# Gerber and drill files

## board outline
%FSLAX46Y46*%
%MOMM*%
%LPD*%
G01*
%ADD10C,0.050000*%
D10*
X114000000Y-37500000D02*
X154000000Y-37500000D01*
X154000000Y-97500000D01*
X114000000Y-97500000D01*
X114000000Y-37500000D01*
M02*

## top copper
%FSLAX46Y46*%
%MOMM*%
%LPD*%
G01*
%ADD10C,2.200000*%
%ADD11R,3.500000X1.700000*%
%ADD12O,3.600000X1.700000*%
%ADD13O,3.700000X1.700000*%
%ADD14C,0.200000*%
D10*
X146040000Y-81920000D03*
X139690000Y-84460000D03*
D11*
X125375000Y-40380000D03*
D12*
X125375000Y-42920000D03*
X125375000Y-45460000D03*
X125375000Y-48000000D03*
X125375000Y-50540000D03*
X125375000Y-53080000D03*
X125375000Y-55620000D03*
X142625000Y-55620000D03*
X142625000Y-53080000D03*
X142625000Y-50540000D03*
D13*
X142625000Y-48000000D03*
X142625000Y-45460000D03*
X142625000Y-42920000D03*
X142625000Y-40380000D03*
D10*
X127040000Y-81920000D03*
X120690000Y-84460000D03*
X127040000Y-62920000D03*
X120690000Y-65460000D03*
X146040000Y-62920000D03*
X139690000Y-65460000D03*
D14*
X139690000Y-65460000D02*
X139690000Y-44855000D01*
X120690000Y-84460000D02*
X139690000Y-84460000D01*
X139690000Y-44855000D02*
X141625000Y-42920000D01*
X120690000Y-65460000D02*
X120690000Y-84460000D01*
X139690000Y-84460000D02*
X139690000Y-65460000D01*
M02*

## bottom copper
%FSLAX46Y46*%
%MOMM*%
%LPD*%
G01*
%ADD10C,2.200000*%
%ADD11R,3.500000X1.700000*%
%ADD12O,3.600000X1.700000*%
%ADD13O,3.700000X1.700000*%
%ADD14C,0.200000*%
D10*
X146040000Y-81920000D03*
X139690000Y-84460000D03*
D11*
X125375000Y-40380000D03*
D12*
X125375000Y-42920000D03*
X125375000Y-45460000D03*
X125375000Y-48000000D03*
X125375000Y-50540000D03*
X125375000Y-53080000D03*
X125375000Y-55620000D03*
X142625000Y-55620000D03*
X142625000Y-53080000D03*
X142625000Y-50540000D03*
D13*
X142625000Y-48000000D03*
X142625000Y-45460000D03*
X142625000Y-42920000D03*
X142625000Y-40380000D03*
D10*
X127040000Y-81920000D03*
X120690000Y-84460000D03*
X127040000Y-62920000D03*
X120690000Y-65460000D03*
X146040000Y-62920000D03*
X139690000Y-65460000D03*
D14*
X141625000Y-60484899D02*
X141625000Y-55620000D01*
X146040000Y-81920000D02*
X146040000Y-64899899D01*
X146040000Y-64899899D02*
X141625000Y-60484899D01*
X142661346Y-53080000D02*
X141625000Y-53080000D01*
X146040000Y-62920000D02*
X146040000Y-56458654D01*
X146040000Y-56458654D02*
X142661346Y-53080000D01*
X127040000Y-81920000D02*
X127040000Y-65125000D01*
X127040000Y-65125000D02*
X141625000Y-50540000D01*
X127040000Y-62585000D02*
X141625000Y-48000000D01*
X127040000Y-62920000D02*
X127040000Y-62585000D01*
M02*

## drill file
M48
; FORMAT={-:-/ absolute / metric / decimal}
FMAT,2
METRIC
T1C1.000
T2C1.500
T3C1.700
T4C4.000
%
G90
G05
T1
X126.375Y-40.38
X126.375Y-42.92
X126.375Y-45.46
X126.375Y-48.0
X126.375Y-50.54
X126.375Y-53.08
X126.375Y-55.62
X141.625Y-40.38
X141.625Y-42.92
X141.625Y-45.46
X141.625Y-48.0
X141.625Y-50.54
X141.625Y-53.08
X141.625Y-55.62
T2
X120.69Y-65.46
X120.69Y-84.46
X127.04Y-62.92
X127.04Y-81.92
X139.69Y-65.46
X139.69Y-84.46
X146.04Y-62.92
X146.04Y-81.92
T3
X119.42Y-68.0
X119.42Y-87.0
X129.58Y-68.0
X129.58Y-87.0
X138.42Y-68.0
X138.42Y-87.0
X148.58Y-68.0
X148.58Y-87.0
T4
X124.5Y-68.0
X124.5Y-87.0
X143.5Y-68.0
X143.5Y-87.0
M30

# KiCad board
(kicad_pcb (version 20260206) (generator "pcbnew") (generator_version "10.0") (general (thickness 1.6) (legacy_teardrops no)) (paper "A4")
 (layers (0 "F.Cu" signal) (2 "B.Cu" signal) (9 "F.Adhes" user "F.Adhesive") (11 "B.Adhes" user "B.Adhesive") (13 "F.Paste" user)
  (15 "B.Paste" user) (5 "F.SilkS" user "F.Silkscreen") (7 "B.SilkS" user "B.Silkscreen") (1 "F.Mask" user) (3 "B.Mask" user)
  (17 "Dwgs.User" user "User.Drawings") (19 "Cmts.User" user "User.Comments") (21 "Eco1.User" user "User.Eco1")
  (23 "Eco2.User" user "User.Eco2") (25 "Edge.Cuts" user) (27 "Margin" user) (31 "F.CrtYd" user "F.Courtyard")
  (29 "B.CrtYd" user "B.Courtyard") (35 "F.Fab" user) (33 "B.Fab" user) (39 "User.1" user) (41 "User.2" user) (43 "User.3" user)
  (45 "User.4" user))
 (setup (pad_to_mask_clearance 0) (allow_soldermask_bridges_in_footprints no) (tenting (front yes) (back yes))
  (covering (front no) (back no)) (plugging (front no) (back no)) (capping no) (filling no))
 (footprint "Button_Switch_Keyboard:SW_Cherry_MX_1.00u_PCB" (layer "F.Cu") (at 146.04 81.92)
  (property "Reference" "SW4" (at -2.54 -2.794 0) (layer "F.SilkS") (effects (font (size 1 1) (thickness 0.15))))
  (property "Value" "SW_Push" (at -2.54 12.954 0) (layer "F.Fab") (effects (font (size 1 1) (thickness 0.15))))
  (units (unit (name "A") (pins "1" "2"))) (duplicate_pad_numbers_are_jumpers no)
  (pad "" np_thru_hole circle (at -7.62 5.08) (size 1.7 1.7) (drill 1.7) (layers "*.Cu" "*.Mask"))
  (pad "" np_thru_hole circle (at -2.54 5.08) (size 4 4) (drill 4) (layers "*.Cu" "*.Mask"))
  (pad "" np_thru_hole circle (at 2.54 5.08) (size 1.7 1.7) (drill 1.7) (layers "*.Cu" "*.Mask"))
  (pad "1" thru_hole circle (at 0 0) (size 2.2 2.2) (drill 1.5) (layers "*.Cu" "*.Mask") (remove_unused_layers no)
   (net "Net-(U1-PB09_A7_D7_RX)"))
  (pad "2" thru_hole circle (at -6.35 2.54) (size 2.2 2.2) (drill 1.5) (layers "*.Cu" "*.Mask") (remove_unused_layers no) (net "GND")))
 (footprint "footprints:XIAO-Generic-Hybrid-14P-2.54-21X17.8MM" (layer "F.Cu") (at 134 48)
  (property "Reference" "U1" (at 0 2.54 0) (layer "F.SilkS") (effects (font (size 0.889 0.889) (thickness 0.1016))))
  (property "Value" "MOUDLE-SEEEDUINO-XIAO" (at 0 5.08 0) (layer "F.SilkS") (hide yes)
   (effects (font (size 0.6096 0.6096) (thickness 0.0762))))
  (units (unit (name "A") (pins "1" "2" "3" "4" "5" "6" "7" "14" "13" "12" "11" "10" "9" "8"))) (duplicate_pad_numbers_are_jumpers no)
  (pad "1" thru_hole rect (at -7.625 -7.62) (size 3.5 1.7) (drill 1 (offset -1 0)) (layers "*.Cu" "*.Mask") (remove_unused_layers no)
   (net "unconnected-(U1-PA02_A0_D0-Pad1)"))
  (pad "2" thru_hole oval (at -7.625 -5.08) (size 3.6 1.7) (drill 1 (offset -1 0)) (layers "*.Cu" "*.Mask") (remove_unused_layers no)
   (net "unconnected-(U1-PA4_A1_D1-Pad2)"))
  (pad "3" thru_hole oval (at -7.625 -2.54) (size 3.6 1.7) (drill 1 (offset -1 0)) (layers "*.Cu" "*.Mask") (remove_unused_layers no)
   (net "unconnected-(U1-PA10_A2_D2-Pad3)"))
  (pad "4" thru_hole oval (at -7.625 0) (size 3.6 1.7) (drill 1 (offset -1 0)) (layers "*.Cu" "*.Mask") (remove_unused_layers no)
   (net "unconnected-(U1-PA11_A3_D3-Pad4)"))
  (pad "5" thru_hole oval (at -7.625 2.54) (size 3.6 1.7) (drill 1 (offset -1 0)) (layers "*.Cu" "*.Mask") (remove_unused_layers no)
   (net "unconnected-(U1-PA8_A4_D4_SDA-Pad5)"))
  (pad "6" thru_hole oval (at -7.625 5.08 180) (size 3.6 1.7) (drill 1 (offset 1 0)) (layers "*.Cu" "*.Mask") (remove_unused_layers no)
   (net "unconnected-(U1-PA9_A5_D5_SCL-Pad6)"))
  (pad "7" thru_hole oval (at -7.625 7.62) (size 3.6 1.7) (drill 1 (offset -1 0)) (layers "*.Cu" "*.Mask") (remove_unused_layers no)
   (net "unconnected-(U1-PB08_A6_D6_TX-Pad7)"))
  (pad "8" thru_hole oval (at 7.625 7.62) (size 3.6 1.7) (drill 1 (offset 1 0)) (layers "*.Cu" "*.Mask") (remove_unused_layers no)
   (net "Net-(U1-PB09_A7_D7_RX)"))
  (pad "9" thru_hole oval (at 7.625 5.08) (size 3.6 1.7) (drill 1 (offset 1 0)) (layers "*.Cu" "*.Mask") (remove_unused_layers no)
   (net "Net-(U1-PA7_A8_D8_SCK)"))
  (pad "10" thru_hole oval (at 7.625 2.54) (size 3.6 1.7) (drill 1 (offset 1 0)) (layers "*.Cu" "*.Mask") (remove_unused_layers no)
   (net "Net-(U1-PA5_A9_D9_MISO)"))
  (pad "11" thru_hole oval (at 7.625 0) (size 3.7 1.7) (drill 1 (offset 1 0)) (layers "*.Cu" "*.Mask") (remove_unused_layers no)
   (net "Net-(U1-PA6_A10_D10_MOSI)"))
  (pad "12" thru_hole oval (at 7.625 -2.54) (size 3.7 1.7) (drill 1 (offset 1 0)) (layers "*.Cu" "*.Mask") (remove_unused_layers no)
   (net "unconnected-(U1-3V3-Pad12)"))
  (pad "13" thru_hole oval (at 7.625 -5.08) (size 3.7 1.7) (drill 1 (offset 1 0)) (layers "*.Cu" "*.Mask") (remove_unused_layers no)
   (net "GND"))
  (pad "14" thru_hole oval (at 7.625 -7.62) (size 3.7 1.7) (drill 1 (offset 1 0)) (layers "*.Cu" "*.Mask") (remove_unused_layers no)
   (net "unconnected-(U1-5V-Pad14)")))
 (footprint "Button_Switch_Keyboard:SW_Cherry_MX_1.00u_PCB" (layer "F.Cu") (at 127.04 81.92)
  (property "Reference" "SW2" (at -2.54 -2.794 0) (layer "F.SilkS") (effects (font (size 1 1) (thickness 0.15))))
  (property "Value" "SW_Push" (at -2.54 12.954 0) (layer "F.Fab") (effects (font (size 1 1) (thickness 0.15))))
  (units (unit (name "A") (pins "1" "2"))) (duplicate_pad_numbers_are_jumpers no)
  (pad "" np_thru_hole circle (at -7.62 5.08) (size 1.7 1.7) (drill 1.7) (layers "*.Cu" "*.Mask"))
  (pad "" np_thru_hole circle (at -2.54 5.08) (size 4 4) (drill 4) (layers "*.Cu" "*.Mask"))
  (pad "" np_thru_hole circle (at 2.54 5.08) (size 1.7 1.7) (drill 1.7) (layers "*.Cu" "*.Mask"))
  (pad "1" thru_hole circle (at 0 0) (size 2.2 2.2) (drill 1.5) (layers "*.Cu" "*.Mask") (remove_unused_layers no)
   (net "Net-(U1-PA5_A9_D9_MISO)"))
  (pad "2" thru_hole circle (at -6.35 2.54) (size 2.2 2.2) (drill 1.5) (layers "*.Cu" "*.Mask") (remove_unused_layers no) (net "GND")))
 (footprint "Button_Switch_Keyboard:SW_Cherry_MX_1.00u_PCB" (layer "F.Cu") (at 127.04 62.92)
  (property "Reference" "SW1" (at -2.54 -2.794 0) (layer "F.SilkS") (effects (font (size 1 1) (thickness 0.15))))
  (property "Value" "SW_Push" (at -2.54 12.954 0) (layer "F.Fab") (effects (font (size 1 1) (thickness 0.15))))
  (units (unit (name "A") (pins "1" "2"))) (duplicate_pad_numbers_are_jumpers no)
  (pad "" np_thru_hole circle (at -7.62 5.08) (size 1.7 1.7) (drill 1.7) (layers "*.Cu" "*.Mask"))
  (pad "" np_thru_hole circle (at -2.54 5.08) (size 4 4) (drill 4) (layers "*.Cu" "*.Mask"))
  (pad "" np_thru_hole circle (at 2.54 5.08) (size 1.7 1.7) (drill 1.7) (layers "*.Cu" "*.Mask"))
  (pad "1" thru_hole circle (at 0 0) (size 2.2 2.2) (drill 1.5) (layers "*.Cu" "*.Mask") (remove_unused_layers no)
   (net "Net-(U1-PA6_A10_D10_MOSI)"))
  (pad "2" thru_hole circle (at -6.35 2.54) (size 2.2 2.2) (drill 1.5) (layers "*.Cu" "*.Mask") (remove_unused_layers no) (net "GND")))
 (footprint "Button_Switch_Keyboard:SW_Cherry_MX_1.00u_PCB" (layer "F.Cu") (at 146.04 62.92)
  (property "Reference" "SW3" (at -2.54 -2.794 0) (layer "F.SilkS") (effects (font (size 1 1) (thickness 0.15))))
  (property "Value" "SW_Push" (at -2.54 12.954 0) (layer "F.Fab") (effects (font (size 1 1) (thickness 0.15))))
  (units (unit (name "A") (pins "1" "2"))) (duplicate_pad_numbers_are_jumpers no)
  (pad "" np_thru_hole circle (at -7.62 5.08) (size 1.7 1.7) (drill 1.7) (layers "*.Cu" "*.Mask"))
  (pad "" np_thru_hole circle (at -2.54 5.08) (size 4 4) (drill 4) (layers "*.Cu" "*.Mask"))
  (pad "" np_thru_hole circle (at 2.54 5.08) (size 1.7 1.7) (drill 1.7) (layers "*.Cu" "*.Mask"))
  (pad "1" thru_hole circle (at 0 0) (size 2.2 2.2) (drill 1.5) (layers "*.Cu" "*.Mask") (remove_unused_layers no)
   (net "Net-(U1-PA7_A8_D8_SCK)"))
  (pad "2" thru_hole circle (at -6.35 2.54) (size 2.2 2.2) (drill 1.5) (layers "*.Cu" "*.Mask") (remove_unused_layers no) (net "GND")))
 (gr_rect (start 114 37.5) (end 154 97.5) (stroke (width 0.05) (type default)) (fill no) (layer "Edge.Cuts"))
 (segment (start 141.625 60.484899) (end 141.625 55.62) (width 0.2) (layer "B.Cu") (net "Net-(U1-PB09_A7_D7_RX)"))
 (segment (start 146.04 81.92) (end 146.04 64.899899) (width 0.2) (layer "B.Cu") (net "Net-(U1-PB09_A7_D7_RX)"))
 (segment (start 146.04 64.899899) (end 141.625 60.484899) (width 0.2) (layer "B.Cu") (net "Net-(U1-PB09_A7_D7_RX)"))
 (segment (start 139.69 65.46) (end 139.69 44.855) (width 0.2) (layer "F.Cu") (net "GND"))
 (segment (start 120.69 84.46) (end 139.69 84.46) (width 0.2) (layer "F.Cu") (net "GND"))
 (segment (start 139.69 44.855) (end 141.625 42.92) (width 0.2) (layer "F.Cu") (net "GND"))
 (segment (start 120.69 65.46) (end 120.69 84.46) (width 0.2) (layer "F.Cu") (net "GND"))
 (segment (start 139.69 84.46) (end 139.69 65.46) (width 0.2) (layer "F.Cu") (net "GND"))
 (segment (start 142.661346 53.08) (end 141.625 53.08) (width 0.2) (layer "B.Cu") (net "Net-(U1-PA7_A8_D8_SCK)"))
 (segment (start 146.04 62.92) (end 146.04 56.458654) (width 0.2) (layer "B.Cu") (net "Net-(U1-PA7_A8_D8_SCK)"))
 (segment (start 146.04 56.458654) (end 142.661346 53.08) (width 0.2) (layer "B.Cu") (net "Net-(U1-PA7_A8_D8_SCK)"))
 (segment (start 127.04 81.92) (end 127.04 65.125) (width 0.2) (layer "B.Cu") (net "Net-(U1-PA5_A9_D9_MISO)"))
 (segment (start 127.04 65.125) (end 141.625 50.54) (width 0.2) (layer "B.Cu") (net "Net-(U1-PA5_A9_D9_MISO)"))
 (segment (start 127.04 62.585) (end 141.625 48) (width 0.2) (layer "B.Cu") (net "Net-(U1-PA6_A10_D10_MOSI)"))
 (segment (start 127.04 62.92) (end 127.04 62.585) (width 0.2) (layer "B.Cu") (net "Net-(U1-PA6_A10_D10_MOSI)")))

